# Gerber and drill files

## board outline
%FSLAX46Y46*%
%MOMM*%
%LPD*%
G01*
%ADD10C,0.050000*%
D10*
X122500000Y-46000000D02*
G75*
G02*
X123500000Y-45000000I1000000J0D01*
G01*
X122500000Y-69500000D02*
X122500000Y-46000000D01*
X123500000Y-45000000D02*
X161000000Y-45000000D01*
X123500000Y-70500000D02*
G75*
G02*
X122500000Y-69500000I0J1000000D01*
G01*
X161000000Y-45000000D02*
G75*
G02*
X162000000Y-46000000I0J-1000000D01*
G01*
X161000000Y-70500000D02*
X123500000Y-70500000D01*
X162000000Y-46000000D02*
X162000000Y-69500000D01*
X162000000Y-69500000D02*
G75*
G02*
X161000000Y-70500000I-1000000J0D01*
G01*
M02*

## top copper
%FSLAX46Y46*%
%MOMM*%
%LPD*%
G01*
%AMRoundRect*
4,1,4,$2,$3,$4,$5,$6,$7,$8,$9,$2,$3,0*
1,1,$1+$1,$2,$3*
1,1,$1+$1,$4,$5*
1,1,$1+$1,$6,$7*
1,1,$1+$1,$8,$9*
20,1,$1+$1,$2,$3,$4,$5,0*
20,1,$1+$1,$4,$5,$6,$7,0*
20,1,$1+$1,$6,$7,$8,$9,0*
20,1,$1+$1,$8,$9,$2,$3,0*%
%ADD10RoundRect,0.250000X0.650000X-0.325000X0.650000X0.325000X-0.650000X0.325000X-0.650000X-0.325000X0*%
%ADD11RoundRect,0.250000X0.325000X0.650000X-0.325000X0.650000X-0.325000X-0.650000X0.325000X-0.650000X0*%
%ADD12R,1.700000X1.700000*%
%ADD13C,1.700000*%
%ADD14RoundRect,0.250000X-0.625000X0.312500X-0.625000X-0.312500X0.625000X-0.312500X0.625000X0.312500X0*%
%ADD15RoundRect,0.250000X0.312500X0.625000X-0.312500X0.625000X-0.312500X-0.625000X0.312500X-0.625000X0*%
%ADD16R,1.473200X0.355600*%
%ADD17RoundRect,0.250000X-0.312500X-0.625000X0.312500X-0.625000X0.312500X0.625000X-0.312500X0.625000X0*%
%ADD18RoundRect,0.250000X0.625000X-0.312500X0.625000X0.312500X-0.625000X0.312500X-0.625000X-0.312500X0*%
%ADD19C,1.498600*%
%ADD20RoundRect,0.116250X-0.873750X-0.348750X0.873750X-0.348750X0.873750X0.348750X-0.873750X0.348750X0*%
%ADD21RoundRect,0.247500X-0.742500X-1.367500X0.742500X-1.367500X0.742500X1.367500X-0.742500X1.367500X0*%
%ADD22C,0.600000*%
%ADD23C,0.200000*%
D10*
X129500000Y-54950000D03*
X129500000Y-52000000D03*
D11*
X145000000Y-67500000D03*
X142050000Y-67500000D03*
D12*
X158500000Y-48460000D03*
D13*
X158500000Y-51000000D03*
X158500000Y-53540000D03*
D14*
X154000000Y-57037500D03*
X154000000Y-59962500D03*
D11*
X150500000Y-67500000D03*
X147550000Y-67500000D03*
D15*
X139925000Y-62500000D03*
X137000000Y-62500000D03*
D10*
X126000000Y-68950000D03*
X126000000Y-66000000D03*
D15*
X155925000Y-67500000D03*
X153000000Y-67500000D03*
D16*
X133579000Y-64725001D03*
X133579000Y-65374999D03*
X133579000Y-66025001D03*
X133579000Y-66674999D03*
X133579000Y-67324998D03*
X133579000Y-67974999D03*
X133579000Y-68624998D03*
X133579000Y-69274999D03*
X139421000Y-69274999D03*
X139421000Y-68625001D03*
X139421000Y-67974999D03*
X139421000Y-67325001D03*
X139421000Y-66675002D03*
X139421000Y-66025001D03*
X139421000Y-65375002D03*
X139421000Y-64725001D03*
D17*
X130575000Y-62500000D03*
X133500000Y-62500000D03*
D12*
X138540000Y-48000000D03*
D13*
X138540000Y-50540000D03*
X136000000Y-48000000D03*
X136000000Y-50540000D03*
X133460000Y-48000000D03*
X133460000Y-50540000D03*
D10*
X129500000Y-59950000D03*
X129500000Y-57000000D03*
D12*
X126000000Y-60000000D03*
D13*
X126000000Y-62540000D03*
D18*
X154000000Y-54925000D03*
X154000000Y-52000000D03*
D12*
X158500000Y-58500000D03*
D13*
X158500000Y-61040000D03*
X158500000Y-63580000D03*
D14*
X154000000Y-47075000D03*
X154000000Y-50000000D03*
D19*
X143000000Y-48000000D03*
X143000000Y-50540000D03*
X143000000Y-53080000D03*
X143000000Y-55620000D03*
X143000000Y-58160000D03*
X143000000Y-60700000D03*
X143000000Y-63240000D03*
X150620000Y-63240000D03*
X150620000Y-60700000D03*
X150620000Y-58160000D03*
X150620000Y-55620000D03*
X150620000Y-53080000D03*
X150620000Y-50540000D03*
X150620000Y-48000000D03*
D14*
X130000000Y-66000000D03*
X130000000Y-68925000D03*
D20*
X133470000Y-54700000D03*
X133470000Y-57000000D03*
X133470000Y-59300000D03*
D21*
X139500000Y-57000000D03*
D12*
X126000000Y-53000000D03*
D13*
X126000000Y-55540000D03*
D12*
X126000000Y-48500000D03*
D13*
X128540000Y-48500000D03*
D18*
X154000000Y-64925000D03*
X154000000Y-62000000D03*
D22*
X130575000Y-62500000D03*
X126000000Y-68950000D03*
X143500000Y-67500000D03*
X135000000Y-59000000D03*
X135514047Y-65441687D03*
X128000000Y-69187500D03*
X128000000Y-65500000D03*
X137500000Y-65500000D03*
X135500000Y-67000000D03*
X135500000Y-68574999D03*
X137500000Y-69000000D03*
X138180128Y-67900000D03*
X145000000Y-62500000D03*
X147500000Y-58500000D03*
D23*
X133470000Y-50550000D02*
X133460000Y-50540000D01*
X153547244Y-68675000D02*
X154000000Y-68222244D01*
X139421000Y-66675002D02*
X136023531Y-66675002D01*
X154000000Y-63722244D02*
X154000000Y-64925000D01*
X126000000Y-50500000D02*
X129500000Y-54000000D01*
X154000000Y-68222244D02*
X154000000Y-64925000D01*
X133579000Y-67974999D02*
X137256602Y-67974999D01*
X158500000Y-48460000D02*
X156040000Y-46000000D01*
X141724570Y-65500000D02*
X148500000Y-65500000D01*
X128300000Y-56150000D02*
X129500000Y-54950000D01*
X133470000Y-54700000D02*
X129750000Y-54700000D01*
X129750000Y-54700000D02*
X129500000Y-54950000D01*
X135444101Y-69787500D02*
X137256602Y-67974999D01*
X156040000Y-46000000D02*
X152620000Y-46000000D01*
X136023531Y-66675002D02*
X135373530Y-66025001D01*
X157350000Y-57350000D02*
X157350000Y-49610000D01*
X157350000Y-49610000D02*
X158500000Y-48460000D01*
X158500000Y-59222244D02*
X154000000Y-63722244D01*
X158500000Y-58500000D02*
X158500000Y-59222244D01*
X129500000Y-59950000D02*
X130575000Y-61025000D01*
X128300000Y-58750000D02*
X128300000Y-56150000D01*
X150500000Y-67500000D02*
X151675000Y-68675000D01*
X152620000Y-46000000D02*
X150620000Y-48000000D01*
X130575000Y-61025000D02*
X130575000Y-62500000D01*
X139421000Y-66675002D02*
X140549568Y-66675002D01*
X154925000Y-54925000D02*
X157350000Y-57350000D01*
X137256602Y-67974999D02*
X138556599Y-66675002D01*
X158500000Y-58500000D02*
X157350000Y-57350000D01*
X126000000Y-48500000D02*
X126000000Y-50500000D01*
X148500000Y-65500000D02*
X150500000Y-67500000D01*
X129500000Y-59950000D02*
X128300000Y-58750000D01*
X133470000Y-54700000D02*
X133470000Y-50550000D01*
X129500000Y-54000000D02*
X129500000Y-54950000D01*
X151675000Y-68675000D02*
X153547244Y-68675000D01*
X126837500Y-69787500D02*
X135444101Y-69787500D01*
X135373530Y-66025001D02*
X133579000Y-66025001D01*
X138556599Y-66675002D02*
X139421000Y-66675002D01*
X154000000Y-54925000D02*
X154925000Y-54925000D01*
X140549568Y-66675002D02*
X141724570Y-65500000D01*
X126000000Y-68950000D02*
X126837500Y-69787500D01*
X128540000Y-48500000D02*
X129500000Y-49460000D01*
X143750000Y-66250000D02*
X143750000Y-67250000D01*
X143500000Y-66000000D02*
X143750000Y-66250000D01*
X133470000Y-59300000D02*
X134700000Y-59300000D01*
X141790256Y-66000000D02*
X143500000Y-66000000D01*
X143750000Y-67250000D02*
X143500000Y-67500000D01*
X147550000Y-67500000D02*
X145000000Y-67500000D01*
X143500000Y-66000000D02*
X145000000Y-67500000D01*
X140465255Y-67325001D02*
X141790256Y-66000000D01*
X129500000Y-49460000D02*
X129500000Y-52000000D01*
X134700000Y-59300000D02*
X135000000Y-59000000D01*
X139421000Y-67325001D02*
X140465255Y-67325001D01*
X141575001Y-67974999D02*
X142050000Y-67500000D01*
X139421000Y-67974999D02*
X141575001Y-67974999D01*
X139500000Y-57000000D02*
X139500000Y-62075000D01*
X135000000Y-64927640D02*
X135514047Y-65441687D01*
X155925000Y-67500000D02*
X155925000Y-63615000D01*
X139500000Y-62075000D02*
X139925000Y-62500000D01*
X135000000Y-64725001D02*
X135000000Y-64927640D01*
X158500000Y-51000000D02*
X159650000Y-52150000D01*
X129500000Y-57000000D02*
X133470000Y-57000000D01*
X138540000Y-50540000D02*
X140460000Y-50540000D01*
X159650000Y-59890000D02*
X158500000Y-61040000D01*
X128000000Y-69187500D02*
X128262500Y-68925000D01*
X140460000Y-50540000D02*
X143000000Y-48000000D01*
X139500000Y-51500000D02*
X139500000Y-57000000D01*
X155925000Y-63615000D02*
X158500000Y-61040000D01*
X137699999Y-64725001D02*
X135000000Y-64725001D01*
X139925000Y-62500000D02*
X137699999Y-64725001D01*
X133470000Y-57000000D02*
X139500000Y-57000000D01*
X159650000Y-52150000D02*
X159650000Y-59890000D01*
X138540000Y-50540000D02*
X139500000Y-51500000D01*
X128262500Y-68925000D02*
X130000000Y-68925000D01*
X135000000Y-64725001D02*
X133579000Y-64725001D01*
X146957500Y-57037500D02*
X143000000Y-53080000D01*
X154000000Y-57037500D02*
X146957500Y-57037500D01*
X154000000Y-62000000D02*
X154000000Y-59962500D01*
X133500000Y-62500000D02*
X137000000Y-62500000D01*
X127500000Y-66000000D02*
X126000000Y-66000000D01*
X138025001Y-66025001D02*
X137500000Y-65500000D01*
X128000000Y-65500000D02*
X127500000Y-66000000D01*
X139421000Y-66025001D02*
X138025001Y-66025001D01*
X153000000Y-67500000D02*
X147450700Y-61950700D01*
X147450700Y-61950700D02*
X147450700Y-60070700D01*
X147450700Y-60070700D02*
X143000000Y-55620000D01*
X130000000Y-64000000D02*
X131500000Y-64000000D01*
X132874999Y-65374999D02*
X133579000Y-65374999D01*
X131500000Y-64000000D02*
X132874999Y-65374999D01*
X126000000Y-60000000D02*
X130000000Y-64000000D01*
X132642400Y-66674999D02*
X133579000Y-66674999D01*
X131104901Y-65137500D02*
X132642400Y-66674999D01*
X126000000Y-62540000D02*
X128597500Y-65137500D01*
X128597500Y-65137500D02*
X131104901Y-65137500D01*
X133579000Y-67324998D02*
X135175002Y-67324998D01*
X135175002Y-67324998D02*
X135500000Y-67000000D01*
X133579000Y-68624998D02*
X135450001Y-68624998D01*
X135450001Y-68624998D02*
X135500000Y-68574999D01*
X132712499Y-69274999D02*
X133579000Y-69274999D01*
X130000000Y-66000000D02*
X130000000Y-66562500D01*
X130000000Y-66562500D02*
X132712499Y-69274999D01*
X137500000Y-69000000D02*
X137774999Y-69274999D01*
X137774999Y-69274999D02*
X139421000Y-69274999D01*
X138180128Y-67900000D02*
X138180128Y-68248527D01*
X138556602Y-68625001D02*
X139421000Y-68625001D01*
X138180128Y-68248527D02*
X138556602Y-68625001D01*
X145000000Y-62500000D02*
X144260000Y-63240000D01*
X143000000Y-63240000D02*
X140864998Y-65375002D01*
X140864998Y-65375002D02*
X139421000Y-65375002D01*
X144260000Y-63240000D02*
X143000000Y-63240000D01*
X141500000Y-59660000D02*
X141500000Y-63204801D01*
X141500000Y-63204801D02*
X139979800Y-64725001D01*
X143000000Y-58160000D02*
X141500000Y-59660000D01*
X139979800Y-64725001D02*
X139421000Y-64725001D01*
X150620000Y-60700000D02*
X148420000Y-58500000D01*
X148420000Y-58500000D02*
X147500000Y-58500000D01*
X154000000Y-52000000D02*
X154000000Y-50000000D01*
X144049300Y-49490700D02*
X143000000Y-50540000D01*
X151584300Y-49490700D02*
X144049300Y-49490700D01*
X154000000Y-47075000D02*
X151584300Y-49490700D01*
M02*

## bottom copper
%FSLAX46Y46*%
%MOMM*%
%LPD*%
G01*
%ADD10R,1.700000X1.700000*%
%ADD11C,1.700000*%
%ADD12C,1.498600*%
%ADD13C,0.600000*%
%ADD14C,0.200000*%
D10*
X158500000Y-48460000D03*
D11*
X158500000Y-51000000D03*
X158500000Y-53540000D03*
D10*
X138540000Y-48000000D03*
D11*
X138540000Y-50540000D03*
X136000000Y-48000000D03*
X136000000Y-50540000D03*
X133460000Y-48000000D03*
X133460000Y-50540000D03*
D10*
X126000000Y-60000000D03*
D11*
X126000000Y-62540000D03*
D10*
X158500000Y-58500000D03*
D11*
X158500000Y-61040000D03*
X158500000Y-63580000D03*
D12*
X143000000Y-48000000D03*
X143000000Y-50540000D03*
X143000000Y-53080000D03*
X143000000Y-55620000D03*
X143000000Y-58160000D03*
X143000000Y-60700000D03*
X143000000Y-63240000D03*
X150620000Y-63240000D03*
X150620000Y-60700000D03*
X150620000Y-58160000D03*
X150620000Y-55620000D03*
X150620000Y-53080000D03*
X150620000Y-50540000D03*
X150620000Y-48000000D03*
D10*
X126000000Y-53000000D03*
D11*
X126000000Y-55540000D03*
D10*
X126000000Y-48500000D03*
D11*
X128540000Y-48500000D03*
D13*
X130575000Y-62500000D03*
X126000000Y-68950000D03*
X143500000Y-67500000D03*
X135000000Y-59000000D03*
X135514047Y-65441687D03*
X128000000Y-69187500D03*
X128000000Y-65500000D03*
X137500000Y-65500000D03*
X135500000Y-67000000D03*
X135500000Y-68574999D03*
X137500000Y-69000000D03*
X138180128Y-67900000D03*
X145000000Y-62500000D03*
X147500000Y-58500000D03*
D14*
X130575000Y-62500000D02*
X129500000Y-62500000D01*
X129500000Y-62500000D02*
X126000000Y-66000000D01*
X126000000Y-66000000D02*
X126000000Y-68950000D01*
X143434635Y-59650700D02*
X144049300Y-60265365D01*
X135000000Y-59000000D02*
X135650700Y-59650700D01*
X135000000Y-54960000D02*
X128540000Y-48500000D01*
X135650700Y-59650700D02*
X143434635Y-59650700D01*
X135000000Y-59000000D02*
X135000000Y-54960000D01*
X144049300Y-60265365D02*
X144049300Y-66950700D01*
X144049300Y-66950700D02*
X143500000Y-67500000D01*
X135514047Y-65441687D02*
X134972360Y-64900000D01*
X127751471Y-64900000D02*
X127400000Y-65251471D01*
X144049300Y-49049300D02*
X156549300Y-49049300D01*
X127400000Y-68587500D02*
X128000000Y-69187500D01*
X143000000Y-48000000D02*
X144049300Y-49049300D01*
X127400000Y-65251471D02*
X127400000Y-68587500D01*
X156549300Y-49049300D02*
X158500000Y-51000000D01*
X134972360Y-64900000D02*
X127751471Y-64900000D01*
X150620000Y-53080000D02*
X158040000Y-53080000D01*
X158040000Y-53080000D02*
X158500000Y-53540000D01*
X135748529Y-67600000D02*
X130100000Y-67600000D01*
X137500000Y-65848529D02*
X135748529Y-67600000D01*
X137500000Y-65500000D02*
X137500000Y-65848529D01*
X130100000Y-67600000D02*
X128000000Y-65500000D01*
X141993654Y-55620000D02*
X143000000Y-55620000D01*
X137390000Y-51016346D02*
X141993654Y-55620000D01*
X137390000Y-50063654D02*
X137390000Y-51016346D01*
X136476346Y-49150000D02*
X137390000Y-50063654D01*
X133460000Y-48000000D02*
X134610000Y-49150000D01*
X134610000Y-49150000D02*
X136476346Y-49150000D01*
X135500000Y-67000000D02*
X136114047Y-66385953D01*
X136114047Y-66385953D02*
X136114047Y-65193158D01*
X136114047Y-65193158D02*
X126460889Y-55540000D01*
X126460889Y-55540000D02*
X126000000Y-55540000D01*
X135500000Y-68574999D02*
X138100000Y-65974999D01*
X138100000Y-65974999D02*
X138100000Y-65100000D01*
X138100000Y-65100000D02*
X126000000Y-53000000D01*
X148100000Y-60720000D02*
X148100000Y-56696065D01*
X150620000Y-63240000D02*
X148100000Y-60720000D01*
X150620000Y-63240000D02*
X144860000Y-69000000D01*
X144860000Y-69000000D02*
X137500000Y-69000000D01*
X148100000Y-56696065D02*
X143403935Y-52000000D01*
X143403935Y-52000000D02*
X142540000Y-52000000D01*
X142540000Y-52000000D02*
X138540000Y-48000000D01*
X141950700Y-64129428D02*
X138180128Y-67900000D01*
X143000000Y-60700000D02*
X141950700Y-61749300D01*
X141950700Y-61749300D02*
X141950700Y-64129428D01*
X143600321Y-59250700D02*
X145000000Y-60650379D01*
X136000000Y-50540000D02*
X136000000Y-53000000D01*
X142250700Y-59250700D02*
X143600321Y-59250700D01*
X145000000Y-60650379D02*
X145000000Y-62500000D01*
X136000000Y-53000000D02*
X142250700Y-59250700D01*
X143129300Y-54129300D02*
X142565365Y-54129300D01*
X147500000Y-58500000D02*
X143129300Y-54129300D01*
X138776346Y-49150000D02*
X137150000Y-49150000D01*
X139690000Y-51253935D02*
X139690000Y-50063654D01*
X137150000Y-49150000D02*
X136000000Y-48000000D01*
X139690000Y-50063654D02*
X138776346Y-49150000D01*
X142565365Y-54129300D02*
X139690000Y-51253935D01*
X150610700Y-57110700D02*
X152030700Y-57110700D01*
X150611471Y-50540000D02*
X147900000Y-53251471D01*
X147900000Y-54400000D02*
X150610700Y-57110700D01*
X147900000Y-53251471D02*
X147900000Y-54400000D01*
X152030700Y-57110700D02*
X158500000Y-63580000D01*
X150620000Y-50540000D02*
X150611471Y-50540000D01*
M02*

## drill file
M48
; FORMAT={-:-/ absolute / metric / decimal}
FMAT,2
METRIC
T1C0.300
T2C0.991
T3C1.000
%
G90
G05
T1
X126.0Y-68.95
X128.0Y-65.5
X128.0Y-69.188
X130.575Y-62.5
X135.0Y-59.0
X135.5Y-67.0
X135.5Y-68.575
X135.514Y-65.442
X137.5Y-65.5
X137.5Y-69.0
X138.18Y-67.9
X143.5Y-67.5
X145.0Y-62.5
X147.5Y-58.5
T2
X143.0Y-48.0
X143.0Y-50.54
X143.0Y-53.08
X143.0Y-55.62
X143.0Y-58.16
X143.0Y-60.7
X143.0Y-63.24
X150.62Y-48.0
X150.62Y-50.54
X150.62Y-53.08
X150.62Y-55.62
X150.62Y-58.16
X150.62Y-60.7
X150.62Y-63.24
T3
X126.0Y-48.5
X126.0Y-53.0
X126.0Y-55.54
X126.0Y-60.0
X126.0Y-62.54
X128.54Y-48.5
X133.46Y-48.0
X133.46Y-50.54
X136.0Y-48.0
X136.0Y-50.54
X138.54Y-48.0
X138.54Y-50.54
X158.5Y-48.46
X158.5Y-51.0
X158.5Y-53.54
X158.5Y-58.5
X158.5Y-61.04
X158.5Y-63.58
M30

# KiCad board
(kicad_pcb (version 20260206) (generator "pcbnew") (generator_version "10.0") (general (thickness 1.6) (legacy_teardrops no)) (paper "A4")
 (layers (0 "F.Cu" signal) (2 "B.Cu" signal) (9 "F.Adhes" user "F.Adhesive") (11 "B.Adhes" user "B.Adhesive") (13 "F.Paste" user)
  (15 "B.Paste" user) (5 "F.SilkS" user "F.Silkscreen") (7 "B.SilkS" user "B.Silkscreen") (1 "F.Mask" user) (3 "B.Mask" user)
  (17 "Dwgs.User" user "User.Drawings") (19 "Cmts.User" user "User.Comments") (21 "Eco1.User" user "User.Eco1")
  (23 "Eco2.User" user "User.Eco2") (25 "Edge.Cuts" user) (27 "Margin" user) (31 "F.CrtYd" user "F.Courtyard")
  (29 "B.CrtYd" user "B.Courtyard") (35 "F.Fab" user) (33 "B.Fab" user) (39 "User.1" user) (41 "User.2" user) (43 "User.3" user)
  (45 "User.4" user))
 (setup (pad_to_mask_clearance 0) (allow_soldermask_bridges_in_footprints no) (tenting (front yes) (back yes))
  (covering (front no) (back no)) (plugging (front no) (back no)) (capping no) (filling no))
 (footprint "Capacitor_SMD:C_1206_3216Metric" (layer "F.Cu") (at 129.5 53.475 90)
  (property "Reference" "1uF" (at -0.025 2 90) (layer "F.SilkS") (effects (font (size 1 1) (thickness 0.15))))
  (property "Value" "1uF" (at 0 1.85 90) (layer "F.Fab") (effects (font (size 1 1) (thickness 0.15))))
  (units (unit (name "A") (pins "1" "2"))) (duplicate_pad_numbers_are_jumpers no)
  (pad "1" smd roundrect (at -1.475 0 90) (size 1.15 1.8) (layers "F.Cu" "F.Mask" "F.Paste") (roundrect_rratio 0.217391) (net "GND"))
  (pad "2" smd roundrect (at 1.475 0 90) (size 1.15 1.8) (layers "F.Cu" "F.Mask" "F.Paste") (roundrect_rratio 0.217391) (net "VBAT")))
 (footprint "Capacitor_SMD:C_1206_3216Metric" (layer "F.Cu") (at 143.525 67.5 180)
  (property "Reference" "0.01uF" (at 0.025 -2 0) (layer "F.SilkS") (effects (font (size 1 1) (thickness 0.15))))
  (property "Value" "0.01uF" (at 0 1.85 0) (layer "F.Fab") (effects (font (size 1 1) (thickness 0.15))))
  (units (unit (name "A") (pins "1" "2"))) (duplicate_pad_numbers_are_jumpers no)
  (pad "1" smd roundrect (at -1.475 0 180) (size 1.15 1.8) (layers "F.Cu" "F.Mask" "F.Paste") (roundrect_rratio 0.217391) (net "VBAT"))
  (pad "2" smd roundrect (at 1.475 0 180) (size 1.15 1.8) (layers "F.Cu" "F.Mask" "F.Paste") (roundrect_rratio 0.217391)
   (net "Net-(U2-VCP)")))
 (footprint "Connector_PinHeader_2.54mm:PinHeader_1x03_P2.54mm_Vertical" (layer "F.Cu") (at 158.5 48.46)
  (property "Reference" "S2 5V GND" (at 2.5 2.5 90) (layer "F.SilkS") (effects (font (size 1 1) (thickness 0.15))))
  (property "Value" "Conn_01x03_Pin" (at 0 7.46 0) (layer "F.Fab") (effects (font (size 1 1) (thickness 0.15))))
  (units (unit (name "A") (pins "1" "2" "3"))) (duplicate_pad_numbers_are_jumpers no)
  (pad "1" thru_hole rect (at 0 0) (size 1.7 1.7) (drill 1) (layers "*.Cu" "*.Mask") (remove_unused_layers no) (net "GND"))
  (pad "2" thru_hole circle (at 0 2.54) (size 1.7 1.7) (drill 1) (layers "*.Cu" "*.Mask") (remove_unused_layers no) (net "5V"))
  (pad "3" thru_hole circle (at 0 5.08) (size 1.7 1.7) (drill 1) (layers "*.Cu" "*.Mask") (remove_unused_layers no)
   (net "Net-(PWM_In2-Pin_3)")))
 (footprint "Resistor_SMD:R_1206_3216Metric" (layer "F.Cu") (at 154 58.5 -90)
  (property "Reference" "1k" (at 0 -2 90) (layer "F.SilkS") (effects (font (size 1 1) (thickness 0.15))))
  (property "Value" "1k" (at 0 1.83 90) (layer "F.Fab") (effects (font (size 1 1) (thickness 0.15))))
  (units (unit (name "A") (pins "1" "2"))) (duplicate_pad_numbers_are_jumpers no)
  (pad "1" smd roundrect (at -1.4625 0 270) (size 1.125 1.75) (layers "F.Cu" "F.Mask" "F.Paste") (roundrect_rratio 0.222222)
   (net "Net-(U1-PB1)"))
  (pad "2" smd roundrect (at 1.4625 0 270) (size 1.125 1.75) (layers "F.Cu" "F.Mask" "F.Paste") (roundrect_rratio 0.222222)
   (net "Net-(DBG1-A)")))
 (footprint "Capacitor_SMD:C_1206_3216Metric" (layer "F.Cu") (at 149.025 67.5 180)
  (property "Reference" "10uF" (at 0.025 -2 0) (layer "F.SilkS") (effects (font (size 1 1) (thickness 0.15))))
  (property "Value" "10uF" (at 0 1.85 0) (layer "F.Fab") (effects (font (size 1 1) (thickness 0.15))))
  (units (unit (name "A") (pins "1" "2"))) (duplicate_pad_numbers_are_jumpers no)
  (pad "1" smd roundrect (at -1.475 0 180) (size 1.15 1.8) (layers "F.Cu" "F.Mask" "F.Paste") (roundrect_rratio 0.217391) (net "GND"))
  (pad "2" smd roundrect (at 1.475 0 180) (size 1.15 1.8) (layers "F.Cu" "F.Mask" "F.Paste") (roundrect_rratio 0.217391) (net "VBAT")))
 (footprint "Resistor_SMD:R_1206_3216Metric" (layer "F.Cu") (at 138.4625 62.5 180)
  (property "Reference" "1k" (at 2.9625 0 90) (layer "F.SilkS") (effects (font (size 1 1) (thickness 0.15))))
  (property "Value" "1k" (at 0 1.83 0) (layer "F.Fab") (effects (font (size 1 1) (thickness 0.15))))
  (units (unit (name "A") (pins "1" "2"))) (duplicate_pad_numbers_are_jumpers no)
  (pad "1" smd roundrect (at -1.4625 0 180) (size 1.125 1.75) (layers "F.Cu" "F.Mask" "F.Paste") (roundrect_rratio 0.222222) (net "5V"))
  (pad "2" smd roundrect (at 1.4625 0 180) (size 1.125 1.75) (layers "F.Cu" "F.Mask" "F.Paste") (roundrect_rratio 0.222222)
   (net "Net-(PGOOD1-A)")))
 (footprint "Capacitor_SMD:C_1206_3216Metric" (layer "F.Cu") (at 126 67.475 90)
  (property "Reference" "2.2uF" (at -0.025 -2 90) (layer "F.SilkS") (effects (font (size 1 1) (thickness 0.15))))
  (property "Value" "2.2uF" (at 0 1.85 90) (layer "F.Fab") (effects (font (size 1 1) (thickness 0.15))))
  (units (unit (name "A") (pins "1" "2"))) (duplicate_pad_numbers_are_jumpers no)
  (pad "1" smd roundrect (at -1.475 0 90) (size 1.15 1.8) (layers "F.Cu" "F.Mask" "F.Paste") (roundrect_rratio 0.217391) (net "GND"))
  (pad "2" smd roundrect (at 1.475 0 90) (size 1.15 1.8) (layers "F.Cu" "F.Mask" "F.Paste") (roundrect_rratio 0.217391)
   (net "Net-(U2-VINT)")))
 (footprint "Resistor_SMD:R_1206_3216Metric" (layer "F.Cu") (at 154.4625 67.5 180)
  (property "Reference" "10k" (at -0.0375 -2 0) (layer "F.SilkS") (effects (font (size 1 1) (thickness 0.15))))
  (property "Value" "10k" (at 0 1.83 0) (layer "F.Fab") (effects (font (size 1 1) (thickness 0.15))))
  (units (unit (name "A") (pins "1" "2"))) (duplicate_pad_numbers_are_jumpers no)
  (pad "1" smd roundrect (at -1.4625 0 180) (size 1.125 1.75) (layers "F.Cu" "F.Mask" "F.Paste") (roundrect_rratio 0.222222) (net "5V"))
  (pad "2" smd roundrect (at 1.4625 0 180) (size 1.125 1.75) (layers "F.Cu" "F.Mask" "F.Paste") (roundrect_rratio 0.222222) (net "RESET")))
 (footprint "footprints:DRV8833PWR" (layer "F.Cu") (at 136.5 67)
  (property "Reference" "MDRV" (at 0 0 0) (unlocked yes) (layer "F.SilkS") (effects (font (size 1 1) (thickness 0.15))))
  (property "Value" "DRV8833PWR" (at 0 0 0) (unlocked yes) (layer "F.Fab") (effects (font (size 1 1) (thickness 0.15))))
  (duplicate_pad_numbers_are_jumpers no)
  (pad "1" smd rect (at -2.921 -2.274999) (size 1.4732 0.3556) (layers "F.Cu" "F.Mask" "F.Paste") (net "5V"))
  (pad "2" smd rect (at -2.921 -1.625001) (size 1.4732 0.3556) (layers "F.Cu" "F.Mask" "F.Paste") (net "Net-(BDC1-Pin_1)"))
  (pad "3" smd rect (at -2.921 -0.974999) (size 1.4732 0.3556) (layers "F.Cu" "F.Mask" "F.Paste") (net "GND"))
  (pad "4" smd rect (at -2.921 -0.325001) (size 1.4732 0.3556) (layers "F.Cu" "F.Mask" "F.Paste") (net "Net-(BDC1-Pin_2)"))
  (pad "5" smd rect (at -2.921 0.324998) (size 1.4732 0.3556) (layers "F.Cu" "F.Mask" "F.Paste") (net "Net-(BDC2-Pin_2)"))
  (pad "6" smd rect (at -2.921 0.974999) (size 1.4732 0.3556) (layers "F.Cu" "F.Mask" "F.Paste") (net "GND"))
  (pad "7" smd rect (at -2.921 1.624998) (size 1.4732 0.3556) (layers "F.Cu" "F.Mask" "F.Paste") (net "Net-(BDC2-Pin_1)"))
  (pad "8" smd rect (at -2.921 2.274999) (size 1.4732 0.3556) (layers "F.Cu" "F.Mask" "F.Paste") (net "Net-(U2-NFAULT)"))
  (pad "9" smd rect (at 2.921 2.274999) (size 1.4732 0.3556) (layers "F.Cu" "F.Mask" "F.Paste") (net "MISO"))
  (pad "10" smd rect (at 2.921 1.625001) (size 1.4732 0.3556) (layers "F.Cu" "F.Mask" "F.Paste") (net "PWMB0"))
  (pad "11" smd rect (at 2.921 0.974999) (size 1.4732 0.3556) (layers "F.Cu" "F.Mask" "F.Paste") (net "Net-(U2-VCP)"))
  (pad "12" smd rect (at 2.921 0.325001) (size 1.4732 0.3556) (layers "F.Cu" "F.Mask" "F.Paste") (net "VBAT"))
  (pad "13" smd rect (at 2.921 -0.324998) (size 1.4732 0.3556) (layers "F.Cu" "F.Mask" "F.Paste") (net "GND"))
  (pad "14" smd rect (at 2.921 -0.974999) (size 1.4732 0.3556) (layers "F.Cu" "F.Mask" "F.Paste") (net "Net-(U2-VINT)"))
  (pad "15" smd rect (at 2.921 -1.624998) (size 1.4732 0.3556) (layers "F.Cu" "F.Mask" "F.Paste") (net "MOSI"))
  (pad "16" smd rect (at 2.921 -2.274999) (size 1.4732 0.3556) (layers "F.Cu" "F.Mask" "F.Paste") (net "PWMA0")))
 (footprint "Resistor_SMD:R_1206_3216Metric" (layer "F.Cu") (at 132.0375 62.5)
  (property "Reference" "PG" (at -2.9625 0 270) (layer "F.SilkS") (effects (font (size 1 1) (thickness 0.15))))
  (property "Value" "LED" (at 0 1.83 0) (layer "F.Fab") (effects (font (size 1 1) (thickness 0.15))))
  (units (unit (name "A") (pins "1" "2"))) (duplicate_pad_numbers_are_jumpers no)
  (pad "1" smd roundrect (at -1.4625 0) (size 1.125 1.75) (layers "F.Cu" "F.Mask" "F.Paste") (roundrect_rratio 0.222222) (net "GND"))
  (pad "2" smd roundrect (at 1.4625 0) (size 1.125 1.75) (layers "F.Cu" "F.Mask" "F.Paste") (roundrect_rratio 0.222222)
   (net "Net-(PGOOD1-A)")))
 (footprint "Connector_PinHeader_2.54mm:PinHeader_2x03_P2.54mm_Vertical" (layer "F.Cu") (at 138.54 48 -90)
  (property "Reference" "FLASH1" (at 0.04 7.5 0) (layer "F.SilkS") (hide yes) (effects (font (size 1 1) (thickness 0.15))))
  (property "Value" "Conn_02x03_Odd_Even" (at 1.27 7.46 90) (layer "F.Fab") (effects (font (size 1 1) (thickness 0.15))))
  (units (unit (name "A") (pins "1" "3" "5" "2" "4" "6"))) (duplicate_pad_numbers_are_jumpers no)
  (pad "1" thru_hole rect (at 0 0 270) (size 1.7 1.7) (drill 1) (layers "*.Cu" "*.Mask") (remove_unused_layers no) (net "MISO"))
  (pad "2" thru_hole circle (at 2.54 0 270) (size 1.7 1.7) (drill 1) (layers "*.Cu" "*.Mask") (remove_unused_layers no) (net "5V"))
  (pad "3" thru_hole circle (at 0 2.54 270) (size 1.7 1.7) (drill 1) (layers "*.Cu" "*.Mask") (remove_unused_layers no) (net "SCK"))
  (pad "4" thru_hole circle (at 2.54 2.54 270) (size 1.7 1.7) (drill 1) (layers "*.Cu" "*.Mask") (remove_unused_layers no) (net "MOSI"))
  (pad "5" thru_hole circle (at 0 5.08 270) (size 1.7 1.7) (drill 1) (layers "*.Cu" "*.Mask") (remove_unused_layers no) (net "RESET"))
  (pad "6" thru_hole circle (at 2.54 5.08 270) (size 1.7 1.7) (drill 1) (layers "*.Cu" "*.Mask") (remove_unused_layers no) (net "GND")))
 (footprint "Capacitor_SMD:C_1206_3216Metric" (layer "F.Cu") (at 129.5 58.475 90)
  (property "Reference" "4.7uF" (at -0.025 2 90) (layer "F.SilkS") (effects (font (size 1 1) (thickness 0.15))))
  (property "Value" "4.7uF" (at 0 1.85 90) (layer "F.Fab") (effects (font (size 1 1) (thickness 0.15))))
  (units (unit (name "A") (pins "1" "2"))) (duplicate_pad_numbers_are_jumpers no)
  (pad "1" smd roundrect (at -1.475 0 90) (size 1.15 1.8) (layers "F.Cu" "F.Mask" "F.Paste") (roundrect_rratio 0.217391) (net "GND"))
  (pad "2" smd roundrect (at 1.475 0 90) (size 1.15 1.8) (layers "F.Cu" "F.Mask" "F.Paste") (roundrect_rratio 0.217391) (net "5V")))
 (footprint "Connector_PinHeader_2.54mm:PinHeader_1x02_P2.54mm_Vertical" (layer "F.Cu") (at 126 60)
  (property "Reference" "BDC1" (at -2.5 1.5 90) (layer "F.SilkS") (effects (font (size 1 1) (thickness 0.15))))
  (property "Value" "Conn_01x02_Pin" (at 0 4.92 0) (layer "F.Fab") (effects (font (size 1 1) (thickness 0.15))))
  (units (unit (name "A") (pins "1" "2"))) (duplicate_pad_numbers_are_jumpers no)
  (pad "1" thru_hole rect (at 0 0) (size 1.7 1.7) (drill 1) (layers "*.Cu" "*.Mask") (remove_unused_layers no) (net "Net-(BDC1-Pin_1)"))
  (pad "2" thru_hole circle (at 0 2.54) (size 1.7 1.7) (drill 1) (layers "*.Cu" "*.Mask") (remove_unused_layers no) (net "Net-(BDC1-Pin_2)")))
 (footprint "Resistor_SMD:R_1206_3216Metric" (layer "F.Cu") (at 154 53.4625 90)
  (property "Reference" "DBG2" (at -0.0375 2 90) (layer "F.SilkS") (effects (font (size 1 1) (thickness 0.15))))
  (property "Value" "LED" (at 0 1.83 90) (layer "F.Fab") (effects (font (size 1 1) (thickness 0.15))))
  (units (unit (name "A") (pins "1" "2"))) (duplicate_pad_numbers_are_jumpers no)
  (pad "1" smd roundrect (at -1.4625 0 90) (size 1.125 1.75) (layers "F.Cu" "F.Mask" "F.Paste") (roundrect_rratio 0.222222) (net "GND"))
  (pad "2" smd roundrect (at 1.4625 0 90) (size 1.125 1.75) (layers "F.Cu" "F.Mask" "F.Paste") (roundrect_rratio 0.222222)
   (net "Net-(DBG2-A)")))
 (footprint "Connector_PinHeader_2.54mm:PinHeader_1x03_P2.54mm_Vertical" (layer "F.Cu") (at 158.5 58.5)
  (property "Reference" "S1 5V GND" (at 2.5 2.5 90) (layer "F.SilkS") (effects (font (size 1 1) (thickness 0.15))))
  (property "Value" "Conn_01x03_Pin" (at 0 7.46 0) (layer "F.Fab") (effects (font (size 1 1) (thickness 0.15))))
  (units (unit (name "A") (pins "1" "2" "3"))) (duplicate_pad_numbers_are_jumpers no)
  (pad "1" thru_hole rect (at 0 0) (size 1.7 1.7) (drill 1) (layers "*.Cu" "*.Mask") (remove_unused_layers no) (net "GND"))
  (pad "2" thru_hole circle (at 0 2.54) (size 1.7 1.7) (drill 1) (layers "*.Cu" "*.Mask") (remove_unused_layers no) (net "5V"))
  (pad "3" thru_hole circle (at 0 5.08) (size 1.7 1.7) (drill 1) (layers "*.Cu" "*.Mask") (remove_unused_layers no)
   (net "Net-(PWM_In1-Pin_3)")))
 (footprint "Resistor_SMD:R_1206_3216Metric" (layer "F.Cu") (at 154 48.5375 -90)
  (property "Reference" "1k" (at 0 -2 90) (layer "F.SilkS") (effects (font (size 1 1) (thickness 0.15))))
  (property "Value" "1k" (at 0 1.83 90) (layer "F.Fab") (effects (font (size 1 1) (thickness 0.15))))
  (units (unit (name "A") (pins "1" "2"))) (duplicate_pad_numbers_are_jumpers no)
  (pad "1" smd roundrect (at -1.4625 0 270) (size 1.125 1.75) (layers "F.Cu" "F.Mask" "F.Paste") (roundrect_rratio 0.222222)
   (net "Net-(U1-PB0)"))
  (pad "2" smd roundrect (at 1.4625 0 270) (size 1.125 1.75) (layers "F.Cu" "F.Mask" "F.Paste") (roundrect_rratio 0.222222)
   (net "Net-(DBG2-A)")))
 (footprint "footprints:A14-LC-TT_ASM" (layer "F.Cu") (at 150.62 48 -90)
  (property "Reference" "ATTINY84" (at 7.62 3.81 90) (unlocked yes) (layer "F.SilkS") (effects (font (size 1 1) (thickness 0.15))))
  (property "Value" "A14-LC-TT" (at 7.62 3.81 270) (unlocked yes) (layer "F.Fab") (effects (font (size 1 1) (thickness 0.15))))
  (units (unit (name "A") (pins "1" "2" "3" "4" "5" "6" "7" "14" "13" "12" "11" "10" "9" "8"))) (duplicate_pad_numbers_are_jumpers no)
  (pad "1" thru_hole circle (at 0 7.62 270) (size 1.4986 1.4986) (drill 0.9906) (layers "*.Cu" "*.Mask") (remove_unused_layers no)
   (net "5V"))
  (pad "2" thru_hole circle (at 2.54 7.62 270) (size 1.4986 1.4986) (drill 0.9906) (layers "*.Cu" "*.Mask") (remove_unused_layers no)
   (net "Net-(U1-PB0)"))
  (pad "3" thru_hole circle (at 5.08 7.62 270) (size 1.4986 1.4986) (drill 0.9906) (layers "*.Cu" "*.Mask") (remove_unused_layers no)
   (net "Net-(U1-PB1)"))
  (pad "4" thru_hole circle (at 7.62 7.62 270) (size 1.4986 1.4986) (drill 0.9906) (layers "*.Cu" "*.Mask") (remove_unused_layers no)
   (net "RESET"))
  (pad "5" thru_hole circle (at 10.16 7.62 270) (size 1.4986 1.4986) (drill 0.9906) (layers "*.Cu" "*.Mask") (remove_unused_layers no)
   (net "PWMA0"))
  (pad "6" thru_hole circle (at 12.7 7.62 270) (size 1.4986 1.4986) (drill 0.9906) (layers "*.Cu" "*.Mask") (remove_unused_layers no)
   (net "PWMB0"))
  (pad "7" thru_hole circle (at 15.24 7.62 270) (size 1.4986 1.4986) (drill 0.9906) (layers "*.Cu" "*.Mask") (remove_unused_layers no)
   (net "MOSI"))
  (pad "8" thru_hole circle (at 15.24 0 270) (size 1.4986 1.4986) (drill 0.9906) (layers "*.Cu" "*.Mask") (remove_unused_layers no)
   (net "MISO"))
  (pad "9" thru_hole circle (at 12.7 0 270) (size 1.4986 1.4986) (drill 0.9906) (layers "*.Cu" "*.Mask") (remove_unused_layers no)
   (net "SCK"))
  (pad "10" thru_hole circle (at 10.16 0 270) (size 1.4986 1.4986) (drill 0.9906) (layers "*.Cu" "*.Mask") (remove_unused_layers no)
   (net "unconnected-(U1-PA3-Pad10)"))
  (pad "11" thru_hole circle (at 7.62 0 270) (size 1.4986 1.4986) (drill 0.9906) (layers "*.Cu" "*.Mask") (remove_unused_layers no)
   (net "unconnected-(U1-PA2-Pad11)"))
  (pad "12" thru_hole circle (at 5.08 0 270) (size 1.4986 1.4986) (drill 0.9906) (layers "*.Cu" "*.Mask") (remove_unused_layers no)
   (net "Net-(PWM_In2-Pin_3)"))
  (pad "13" thru_hole circle (at 2.54 0 270) (size 1.4986 1.4986) (drill 0.9906) (layers "*.Cu" "*.Mask") (remove_unused_layers no)
   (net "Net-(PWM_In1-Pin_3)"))
  (pad "14" thru_hole circle (at 0 0 270) (size 1.4986 1.4986) (drill 0.9906) (layers "*.Cu" "*.Mask") (remove_unused_layers no) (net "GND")))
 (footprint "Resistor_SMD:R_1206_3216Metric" (layer "F.Cu") (at 130 67.4625 -90)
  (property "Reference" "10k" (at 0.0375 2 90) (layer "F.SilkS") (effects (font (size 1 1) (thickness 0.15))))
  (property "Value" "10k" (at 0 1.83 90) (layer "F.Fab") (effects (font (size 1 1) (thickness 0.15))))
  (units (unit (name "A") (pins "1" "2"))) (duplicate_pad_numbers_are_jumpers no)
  (pad "1" smd roundrect (at -1.4625 0 270) (size 1.125 1.75) (layers "F.Cu" "F.Mask" "F.Paste") (roundrect_rratio 0.222222)
   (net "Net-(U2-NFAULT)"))
  (pad "2" smd roundrect (at 1.4625 0 270) (size 1.125 1.75) (layers "F.Cu" "F.Mask" "F.Paste") (roundrect_rratio 0.222222) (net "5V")))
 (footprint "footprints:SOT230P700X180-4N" (layer "F.Cu") (at 136.485 57)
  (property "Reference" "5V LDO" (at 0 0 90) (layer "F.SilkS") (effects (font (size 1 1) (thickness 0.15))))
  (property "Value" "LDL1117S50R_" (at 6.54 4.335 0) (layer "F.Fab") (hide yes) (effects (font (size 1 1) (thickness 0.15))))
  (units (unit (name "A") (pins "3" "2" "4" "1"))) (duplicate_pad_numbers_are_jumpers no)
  (pad "1" smd roundrect (at -3.015 -2.3) (size 1.98 0.93) (layers "F.Cu" "F.Mask" "F.Paste") (roundrect_rratio 0.125) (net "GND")
   (solder_mask_margin 0.102))
  (pad "2" smd roundrect (at -3.015 0) (size 1.98 0.93) (layers "F.Cu" "F.Mask" "F.Paste") (roundrect_rratio 0.125) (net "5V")
   (solder_mask_margin 0.102))
  (pad "3" smd roundrect (at -3.015 2.3) (size 1.98 0.93) (layers "F.Cu" "F.Mask" "F.Paste") (roundrect_rratio 0.125) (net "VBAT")
   (solder_mask_margin 0.102))
  (pad "4" smd roundrect (at 3.015 0) (size 1.98 3.23) (layers "F.Cu" "F.Mask" "F.Paste") (roundrect_rratio 0.125) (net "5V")
   (solder_mask_margin 0.102)))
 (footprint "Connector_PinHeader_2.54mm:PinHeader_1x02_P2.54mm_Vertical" (layer "F.Cu") (at 126 53)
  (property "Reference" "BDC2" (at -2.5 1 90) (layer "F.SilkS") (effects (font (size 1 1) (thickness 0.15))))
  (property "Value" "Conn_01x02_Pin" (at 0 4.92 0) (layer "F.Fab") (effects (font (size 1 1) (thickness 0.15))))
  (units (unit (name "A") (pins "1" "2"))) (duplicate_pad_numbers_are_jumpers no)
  (pad "1" thru_hole rect (at 0 0) (size 1.7 1.7) (drill 1) (layers "*.Cu" "*.Mask") (remove_unused_layers no) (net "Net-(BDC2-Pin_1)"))
  (pad "2" thru_hole circle (at 0 2.54) (size 1.7 1.7) (drill 1) (layers "*.Cu" "*.Mask") (remove_unused_layers no) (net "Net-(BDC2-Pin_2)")))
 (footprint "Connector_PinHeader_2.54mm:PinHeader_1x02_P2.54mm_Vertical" (layer "F.Cu") (at 126 48.5 90)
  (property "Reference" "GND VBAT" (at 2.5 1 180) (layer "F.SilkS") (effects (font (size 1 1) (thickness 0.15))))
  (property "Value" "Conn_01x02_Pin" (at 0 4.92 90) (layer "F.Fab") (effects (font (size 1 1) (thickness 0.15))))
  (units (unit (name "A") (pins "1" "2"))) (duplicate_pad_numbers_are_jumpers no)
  (pad "1" thru_hole rect (at 0 0 90) (size 1.7 1.7) (drill 1) (layers "*.Cu" "*.Mask") (remove_unused_layers no) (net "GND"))
  (pad "2" thru_hole circle (at 0 2.54 90) (size 1.7 1.7) (drill 1) (layers "*.Cu" "*.Mask") (remove_unused_layers no) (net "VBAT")))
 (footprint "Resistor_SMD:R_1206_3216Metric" (layer "F.Cu") (at 154 63.4625 90)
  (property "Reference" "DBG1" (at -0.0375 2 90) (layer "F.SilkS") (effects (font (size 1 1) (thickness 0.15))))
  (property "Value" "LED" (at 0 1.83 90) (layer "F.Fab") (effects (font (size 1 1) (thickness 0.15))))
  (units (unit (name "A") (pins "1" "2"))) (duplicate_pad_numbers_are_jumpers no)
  (pad "1" smd roundrect (at -1.4625 0 90) (size 1.125 1.75) (layers "F.Cu" "F.Mask" "F.Paste") (roundrect_rratio 0.222222) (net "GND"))
  (pad "2" smd roundrect (at 1.4625 0 90) (size 1.125 1.75) (layers "F.Cu" "F.Mask" "F.Paste") (roundrect_rratio 0.222222)
   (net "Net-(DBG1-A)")))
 (gr_arc (start 122.5 46) (mid 122.792893 45.292893) (end 123.5 45) (stroke (width 0.05) (type default)) (layer "Edge.Cuts"))
 (gr_line (start 122.5 69.5) (end 122.5 46) (stroke (width 0.05) (type default)) (layer "Edge.Cuts"))
 (gr_line (start 123.5 45) (end 161 45) (stroke (width 0.05) (type default)) (layer "Edge.Cuts"))
 (gr_arc (start 123.5 70.5) (mid 122.792893 70.207107) (end 122.5 69.5) (stroke (width 0.05) (type default)) (layer "Edge.Cuts"))
 (gr_arc (start 161 45) (mid 161.707107 45.292893) (end 162 46) (stroke (width 0.05) (type default)) (layer "Edge.Cuts"))
 (gr_line (start 161 70.5) (end 123.5 70.5) (stroke (width 0.05) (type default)) (layer "Edge.Cuts"))
 (gr_line (start 162 46) (end 162 69.5) (stroke (width 0.05) (type default)) (layer "Edge.Cuts"))
 (gr_arc (start 162 69.5) (mid 161.707107 70.207107) (end 161 70.5) (stroke (width 0.05) (type default)) (layer "Edge.Cuts"))
 (segment (start 133.47 50.55) (end 133.46 50.54) (width 0.2) (layer "F.Cu") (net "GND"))
 (segment (start 153.547244 68.675) (end 154 68.222244) (width 0.2) (layer "F.Cu") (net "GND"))
 (segment (start 139.421 66.675002) (end 136.023531 66.675002) (width 0.2) (layer "F.Cu") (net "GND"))
 (segment (start 154 63.722244) (end 154 64.925) (width 0.2) (layer "F.Cu") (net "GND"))
 (segment (start 126 50.5) (end 129.5 54) (width 0.2) (layer "F.Cu") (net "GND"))
 (segment (start 154 68.222244) (end 154 64.925) (width 0.2) (layer "F.Cu") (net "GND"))
 (segment (start 133.579 67.974999) (end 137.256602 67.974999) (width 0.2) (layer "F.Cu") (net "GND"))
 (segment (start 158.5 48.46) (end 156.04 46) (width 0.2) (layer "F.Cu") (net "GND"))
 (segment (start 141.72457 65.5) (end 148.5 65.5) (width 0.2) (layer "F.Cu") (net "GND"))
 (segment (start 128.3 56.15) (end 129.5 54.95) (width 0.2) (layer "F.Cu") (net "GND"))
 (segment (start 133.47 54.7) (end 129.75 54.7) (width 0.2) (layer "F.Cu") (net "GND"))
 (segment (start 129.75 54.7) (end 129.5 54.95) (width 0.2) (layer "F.Cu") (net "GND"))
 (segment (start 135.444101 69.7875) (end 137.256602 67.974999) (width 0.2) (layer "F.Cu") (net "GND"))
 (segment (start 156.04 46) (end 152.62 46) (width 0.2) (layer "F.Cu") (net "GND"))
 (segment (start 136.023531 66.675002) (end 135.37353 66.025001) (width 0.2) (layer "F.Cu") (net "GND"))
 (segment (start 157.35 57.35) (end 157.35 49.61) (width 0.2) (layer "F.Cu") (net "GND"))
 (segment (start 157.35 49.61) (end 158.5 48.46) (width 0.2) (layer "F.Cu") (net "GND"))
 (segment (start 158.5 59.222244) (end 154 63.722244) (width 0.2) (layer "F.Cu") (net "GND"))
 (segment (start 158.5 58.5) (end 158.5 59.222244) (width 0.2) (layer "F.Cu") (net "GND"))
 (segment (start 129.5 59.95) (end 130.575 61.025) (width 0.2) (layer "F.Cu") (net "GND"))
 (segment (start 128.3 58.75) (end 128.3 56.15) (width 0.2) (layer "F.Cu") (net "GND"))
 (segment (start 150.5 67.5) (end 151.675 68.675) (width 0.2) (layer "F.Cu") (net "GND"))
 (segment (start 152.62 46) (end 150.62 48) (width 0.2) (layer "F.Cu") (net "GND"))
 (segment (start 130.575 61.025) (end 130.575 62.5) (width 0.2) (layer "F.Cu") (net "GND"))
 (segment (start 139.421 66.675002) (end 140.549568 66.675002) (width 0.2) (layer "F.Cu") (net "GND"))
 (segment (start 154.925 54.925) (end 157.35 57.35) (width 0.2) (layer "F.Cu") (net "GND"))
 (segment (start 137.256602 67.974999) (end 138.556599 66.675002) (width 0.2) (layer "F.Cu") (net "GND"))
 (segment (start 158.5 58.5) (end 157.35 57.35) (width 0.2) (layer "F.Cu") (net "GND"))
 (segment (start 126 48.5) (end 126 50.5) (width 0.2) (layer "F.Cu") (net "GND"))
 (segment (start 148.5 65.5) (end 150.5 67.5) (width 0.2) (layer "F.Cu") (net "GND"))
 (segment (start 129.5 59.95) (end 128.3 58.75) (width 0.2) (layer "F.Cu") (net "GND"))
 (segment (start 133.47 54.7) (end 133.47 50.55) (width 0.2) (layer "F.Cu") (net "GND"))
 (segment (start 129.5 54) (end 129.5 54.95) (width 0.2) (layer "F.Cu") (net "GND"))
 (segment (start 151.675 68.675) (end 153.547244 68.675) (width 0.2) (layer "F.Cu") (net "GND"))
 (segment (start 126.8375 69.7875) (end 135.444101 69.7875) (width 0.2) (layer "F.Cu") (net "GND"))
 (segment (start 135.37353 66.025001) (end 133.579 66.025001) (width 0.2) (layer "F.Cu") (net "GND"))
 (segment (start 138.556599 66.675002) (end 139.421 66.675002) (width 0.2) (layer "F.Cu") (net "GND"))
 (segment (start 154 54.925) (end 154.925 54.925) (width 0.2) (layer "F.Cu") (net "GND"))
 (segment (start 140.549568 66.675002) (end 141.72457 65.5) (width 0.2) (layer "F.Cu") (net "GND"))
 (segment (start 126 68.95) (end 126.8375 69.7875) (width 0.2) (layer "F.Cu") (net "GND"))
 (via (at 130.575 62.5) (size 0.6) (drill 0.3) (layers "F.Cu" "B.Cu") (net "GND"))
 (via (at 126 68.95) (size 0.6) (drill 0.3) (layers "F.Cu" "B.Cu") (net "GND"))
 (segment (start 130.575 62.5) (end 129.5 62.5) (width 0.2) (layer "B.Cu") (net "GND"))
 (segment (start 129.5 62.5) (end 126 66) (width 0.2) (layer "B.Cu") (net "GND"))
 (segment (start 126 66) (end 126 68.95) (width 0.2) (layer "B.Cu") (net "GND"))
 (segment (start 128.54 48.5) (end 129.5 49.46) (width 0.2) (layer "F.Cu") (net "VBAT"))
 (segment (start 143.75 66.25) (end 143.75 67.25) (width 0.2) (layer "F.Cu") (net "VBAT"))
 (segment (start 143.5 66) (end 143.75 66.25) (width 0.2) (layer "F.Cu") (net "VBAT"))
 (segment (start 133.47 59.3) (end 134.7 59.3) (width 0.2) (layer "F.Cu") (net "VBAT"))
 (segment (start 141.790256 66) (end 143.5 66) (width 0.2) (layer "F.Cu") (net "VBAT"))
 (segment (start 143.75 67.25) (end 143.5 67.5) (width 0.2) (layer "F.Cu") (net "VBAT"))
 (segment (start 147.55 67.5) (end 145 67.5) (width 0.2) (layer "F.Cu") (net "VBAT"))
 (segment (start 143.5 66) (end 145 67.5) (width 0.2) (layer "F.Cu") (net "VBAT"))
 (segment (start 140.465255 67.325001) (end 141.790256 66) (width 0.2) (layer "F.Cu") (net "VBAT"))
 (segment (start 129.5 49.46) (end 129.5 52) (width 0.2) (layer "F.Cu") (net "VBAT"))
 (segment (start 134.7 59.3) (end 135 59) (width 0.2) (layer "F.Cu") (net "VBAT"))
 (segment (start 139.421 67.325001) (end 140.465255 67.325001) (width 0.2) (layer "F.Cu") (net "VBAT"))
 (via (at 143.5 67.5) (size 0.6) (drill 0.3) (layers "F.Cu" "B.Cu") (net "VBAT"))
 (via (at 135 59) (size 0.6) (drill 0.3) (layers "F.Cu" "B.Cu") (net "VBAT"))
 (segment (start 143.434635 59.6507) (end 144.0493 60.265365) (width 0.2) (layer "B.Cu") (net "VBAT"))
 (segment (start 135 59) (end 135.6507 59.6507) (width 0.2) (layer "B.Cu") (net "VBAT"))
 (segment (start 135 54.96) (end 128.54 48.5) (width 0.2) (layer "B.Cu") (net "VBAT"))
 (segment (start 135.6507 59.6507) (end 143.434635 59.6507) (width 0.2) (layer "B.Cu") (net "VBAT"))
 (segment (start 135 59) (end 135 54.96) (width 0.2) (layer "B.Cu") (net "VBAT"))
 (segment (start 144.0493 60.265365) (end 144.0493 66.9507) (width 0.2) (layer "B.Cu") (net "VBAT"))
 (segment (start 144.0493 66.9507) (end 143.5 67.5) (width 0.2) (layer "B.Cu") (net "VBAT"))
 (segment (start 141.575001 67.974999) (end 142.05 67.5) (width 0.2) (layer "F.Cu") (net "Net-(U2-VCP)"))
 (segment (start 139.421 67.974999) (end 141.575001 67.974999) (width 0.2) (layer "F.Cu") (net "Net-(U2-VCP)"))
 (segment (start 139.5 57) (end 139.5 62.075) (width 0.2) (layer "F.Cu") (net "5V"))
 (segment (start 135 64.92764) (end 135.514047 65.441687) (width 0.2) (layer "F.Cu") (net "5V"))
 (segment (start 155.925 67.5) (end 155.925 63.615) (width 0.2) (layer "F.Cu") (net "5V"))
 (segment (start 139.5 62.075) (end 139.925 62.5) (width 0.2) (layer "F.Cu") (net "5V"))
 (segment (start 135 64.725001) (end 135 64.92764) (width 0.2) (layer "F.Cu") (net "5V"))
 (segment (start 158.5 51) (end 159.65 52.15) (width 0.2) (layer "F.Cu") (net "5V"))
 (segment (start 129.5 57) (end 133.47 57) (width 0.2) (layer "F.Cu") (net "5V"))
 (segment (start 138.54 50.54) (end 140.46 50.54) (width 0.2) (layer "F.Cu") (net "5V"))
 (segment (start 159.65 59.89) (end 158.5 61.04) (width 0.2) (layer "F.Cu") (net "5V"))
 (segment (start 128 69.1875) (end 128.2625 68.925) (width 0.2) (layer "F.Cu") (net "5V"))
 (segment (start 140.46 50.54) (end 143 48) (width 0.2) (layer "F.Cu") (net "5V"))
 (segment (start 139.5 51.5) (end 139.5 57) (width 0.2) (layer "F.Cu") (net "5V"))
 (segment (start 155.925 63.615) (end 158.5 61.04) (width 0.2) (layer "F.Cu") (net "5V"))
 (segment (start 137.699999 64.725001) (end 135 64.725001) (width 0.2) (layer "F.Cu") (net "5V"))
 (segment (start 139.925 62.5) (end 137.699999 64.725001) (width 0.2) (layer "F.Cu") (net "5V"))
 (segment (start 133.47 57) (end 139.5 57) (width 0.2) (layer "F.Cu") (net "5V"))
 (segment (start 159.65 52.15) (end 159.65 59.89) (width 0.2) (layer "F.Cu") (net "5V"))
 (segment (start 138.54 50.54) (end 139.5 51.5) (width 0.2) (layer "F.Cu") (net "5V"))
 (segment (start 128.2625 68.925) (end 130 68.925) (width 0.2) (layer "F.Cu") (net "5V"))
 (segment (start 135 64.725001) (end 133.579 64.725001) (width 0.2) (layer "F.Cu") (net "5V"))
 (via (at 135.514047 65.441687) (size 0.6) (drill 0.3) (layers "F.Cu" "B.Cu") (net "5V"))
 (via (at 128 69.1875) (size 0.6) (drill 0.3) (layers "F.Cu" "B.Cu") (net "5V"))
 (segment (start 135.514047 65.441687) (end 134.97236 64.9) (width 0.2) (layer "B.Cu") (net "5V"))
 (segment (start 127.751471 64.9) (end 127.4 65.251471) (width 0.2) (layer "B.Cu") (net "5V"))
 (segment (start 144.0493 49.0493) (end 156.5493 49.0493) (width 0.2) (layer "B.Cu") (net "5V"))
 (segment (start 127.4 68.5875) (end 128 69.1875) (width 0.2) (layer "B.Cu") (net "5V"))
 (segment (start 143 48) (end 144.0493 49.0493) (width 0.2) (layer "B.Cu") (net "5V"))
 (segment (start 127.4 65.251471) (end 127.4 68.5875) (width 0.2) (layer "B.Cu") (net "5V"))
 (segment (start 156.5493 49.0493) (end 158.5 51) (width 0.2) (layer "B.Cu") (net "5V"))
 (segment (start 134.97236 64.9) (end 127.751471 64.9) (width 0.2) (layer "B.Cu") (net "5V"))
 (segment (start 150.62 53.08) (end 158.04 53.08) (width 0.2) (layer "B.Cu") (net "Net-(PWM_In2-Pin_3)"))
 (segment (start 158.04 53.08) (end 158.5 53.54) (width 0.2) (layer "B.Cu") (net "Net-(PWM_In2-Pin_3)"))
 (segment (start 146.9575 57.0375) (end 143 53.08) (width 0.2) (layer "F.Cu") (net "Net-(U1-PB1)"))
 (segment (start 154 57.0375) (end 146.9575 57.0375) (width 0.2) (layer "F.Cu") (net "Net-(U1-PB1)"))
 (segment (start 154 62) (end 154 59.9625) (width 0.2) (layer "F.Cu") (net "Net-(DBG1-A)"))
 (segment (start 133.5 62.5) (end 137 62.5) (width 0.2) (layer "F.Cu") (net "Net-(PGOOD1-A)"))
 (segment (start 127.5 66) (end 126 66) (width 0.2) (layer "F.Cu") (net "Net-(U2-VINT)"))
 (segment (start 138.025001 66.025001) (end 137.5 65.5) (width 0.2) (layer "F.Cu") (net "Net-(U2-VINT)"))
 (segment (start 128 65.5) (end 127.5 66) (width 0.2) (layer "F.Cu") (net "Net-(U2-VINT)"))
 (segment (start 139.421 66.025001) (end 138.025001 66.025001) (width 0.2) (layer "F.Cu") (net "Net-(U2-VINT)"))
 (via (at 128 65.5) (size 0.6) (drill 0.3) (layers "F.Cu" "B.Cu") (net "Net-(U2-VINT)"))
 (via (at 137.5 65.5) (size 0.6) (drill 0.3) (layers "F.Cu" "B.Cu") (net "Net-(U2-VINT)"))
 (segment (start 135.748529 67.6) (end 130.1 67.6) (width 0.2) (layer "B.Cu") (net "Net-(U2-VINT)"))
 (segment (start 137.5 65.848529) (end 135.748529 67.6) (width 0.2) (layer "B.Cu") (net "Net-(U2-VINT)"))
 (segment (start 137.5 65.5) (end 137.5 65.848529) (width 0.2) (layer "B.Cu") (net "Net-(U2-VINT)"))
 (segment (start 130.1 67.6) (end 128 65.5) (width 0.2) (layer "B.Cu") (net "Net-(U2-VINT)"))
 (segment (start 153 67.5) (end 147.4507 61.9507) (width 0.2) (layer "F.Cu") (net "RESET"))
 (segment (start 147.4507 61.9507) (end 147.4507 60.0707) (width 0.2) (layer "F.Cu") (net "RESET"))
 (segment (start 147.4507 60.0707) (end 143 55.62) (width 0.2) (layer "F.Cu") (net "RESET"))
 (segment (start 141.993654 55.62) (end 143 55.62) (width 0.2) (layer "B.Cu") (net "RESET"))
 (segment (start 137.39 51.016346) (end 141.993654 55.62) (width 0.2) (layer "B.Cu") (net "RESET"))
 (segment (start 137.39 50.063654) (end 137.39 51.016346) (width 0.2) (layer "B.Cu") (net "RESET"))
 (segment (start 136.476346 49.15) (end 137.39 50.063654) (width 0.2) (layer "B.Cu") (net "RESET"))
 (segment (start 133.46 48) (end 134.61 49.15) (width 0.2) (layer "B.Cu") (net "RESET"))
 (segment (start 134.61 49.15) (end 136.476346 49.15) (width 0.2) (layer "B.Cu") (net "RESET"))
 (segment (start 130 64) (end 131.5 64) (width 0.2) (layer "F.Cu") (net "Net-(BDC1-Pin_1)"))
 (segment (start 132.874999 65.374999) (end 133.579 65.374999) (width 0.2) (layer "F.Cu") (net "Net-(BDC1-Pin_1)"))
 (segment (start 131.5 64) (end 132.874999 65.374999) (width 0.2) (layer "F.Cu") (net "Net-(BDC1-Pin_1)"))
 (segment (start 126 60) (end 130 64) (width 0.2) (layer "F.Cu") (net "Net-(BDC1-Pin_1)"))
 (segment (start 132.6424 66.674999) (end 133.579 66.674999) (width 0.2) (layer "F.Cu") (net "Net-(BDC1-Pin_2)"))
 (segment (start 131.104901 65.1375) (end 132.6424 66.674999) (width 0.2) (layer "F.Cu") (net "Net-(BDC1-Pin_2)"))
 (segment (start 126 62.54) (end 128.5975 65.1375) (width 0.2) (layer "F.Cu") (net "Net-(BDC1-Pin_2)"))
 (segment (start 128.5975 65.1375) (end 131.104901 65.1375) (width 0.2) (layer "F.Cu") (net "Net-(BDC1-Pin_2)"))
 (segment (start 133.579 67.324998) (end 135.175002 67.324998) (width 0.2) (layer "F.Cu") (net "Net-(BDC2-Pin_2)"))
 (segment (start 135.175002 67.324998) (end 135.5 67) (width 0.2) (layer "F.Cu") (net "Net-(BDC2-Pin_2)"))
 (via (at 135.5 67) (size 0.6) (drill 0.3) (layers "F.Cu" "B.Cu") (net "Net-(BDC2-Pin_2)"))
 (segment (start 135.5 67) (end 136.114047 66.385953) (width 0.2) (layer "B.Cu") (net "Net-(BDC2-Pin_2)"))
 (segment (start 136.114047 66.385953) (end 136.114047 65.193158) (width 0.2) (layer "B.Cu") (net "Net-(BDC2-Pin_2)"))
 (segment (start 136.114047 65.193158) (end 126.460889 55.54) (width 0.2) (layer "B.Cu") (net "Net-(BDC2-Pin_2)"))
 (segment (start 126.460889 55.54) (end 126 55.54) (width 0.2) (layer "B.Cu") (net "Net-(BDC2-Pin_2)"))
 (segment (start 133.579 68.624998) (end 135.450001 68.624998) (width 0.2) (layer "F.Cu") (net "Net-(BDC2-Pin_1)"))
 (segment (start 135.450001 68.624998) (end 135.5 68.574999) (width 0.2) (layer "F.Cu") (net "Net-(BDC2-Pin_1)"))
 (via (at 135.5 68.574999) (size 0.6) (drill 0.3) (layers "F.Cu" "B.Cu") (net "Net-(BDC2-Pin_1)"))
 (segment (start 135.5 68.574999) (end 138.1 65.974999) (width 0.2) (layer "B.Cu") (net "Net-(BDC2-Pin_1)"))
 (segment (start 138.1 65.974999) (end 138.1 65.1) (width 0.2) (layer "B.Cu") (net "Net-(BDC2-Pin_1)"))
 (segment (start 138.1 65.1) (end 126 53) (width 0.2) (layer "B.Cu") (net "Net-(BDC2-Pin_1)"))
 (segment (start 132.712499 69.274999) (end 133.579 69.274999) (width 0.2) (layer "F.Cu") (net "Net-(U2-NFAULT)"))
 (segment (start 130 66) (end 130 66.5625) (width 0.2) (layer "F.Cu") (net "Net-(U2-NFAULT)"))
 (segment (start 130 66.5625) (end 132.712499 69.274999) (width 0.2) (layer "F.Cu") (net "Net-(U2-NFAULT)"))
 (segment (start 137.5 69) (end 137.774999 69.274999) (width 0.2) (layer "F.Cu") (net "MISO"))
 (segment (start 137.774999 69.274999) (end 139.421 69.274999) (width 0.2) (layer "F.Cu") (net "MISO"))
 (via (at 137.5 69) (size 0.6) (drill 0.3) (layers "F.Cu" "B.Cu") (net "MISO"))
 (segment (start 148.1 60.72) (end 148.1 56.696065) (width 0.2) (layer "B.Cu") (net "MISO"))
 (segment (start 150.62 63.24) (end 148.1 60.72) (width 0.2) (layer "B.Cu") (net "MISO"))
 (segment (start 150.62 63.24) (end 144.86 69) (width 0.2) (layer "B.Cu") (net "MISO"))
 (segment (start 144.86 69) (end 137.5 69) (width 0.2) (layer "B.Cu") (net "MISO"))
 (segment (start 148.1 56.696065) (end 143.403935 52) (width 0.2) (layer "B.Cu") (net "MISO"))
 (segment (start 143.403935 52) (end 142.54 52) (width 0.2) (layer "B.Cu") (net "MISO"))
 (segment (start 142.54 52) (end 138.54 48) (width 0.2) (layer "B.Cu") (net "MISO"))
 (segment (start 138.180128 67.9) (end 138.180128 68.248527) (width 0.2) (layer "F.Cu") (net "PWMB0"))
 (segment (start 138.556602 68.625001) (end 139.421 68.625001) (width 0.2) (layer "F.Cu") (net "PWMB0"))
 (segment (start 138.180128 68.248527) (end 138.556602 68.625001) (width 0.2) (layer "F.Cu") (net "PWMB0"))
 (via (at 138.180128 67.9) (size 0.6) (drill 0.3) (layers "F.Cu" "B.Cu") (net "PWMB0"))
 (segment (start 141.9507 64.129428) (end 138.180128 67.9) (width 0.2) (layer "B.Cu") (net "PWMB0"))
 (segment (start 143 60.7) (end 141.9507 61.7493) (width 0.2) (layer "B.Cu") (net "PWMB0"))
 (segment (start 141.9507 61.7493) (end 141.9507 64.129428) (width 0.2) (layer "B.Cu") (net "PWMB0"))
 (segment (start 145 62.5) (end 144.26 63.24) (width 0.2) (layer "F.Cu") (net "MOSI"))
 (segment (start 143 63.24) (end 140.864998 65.375002) (width 0.2) (layer "F.Cu") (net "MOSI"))
 (segment (start 140.864998 65.375002) (end 139.421 65.375002) (width 0.2) (layer "F.Cu") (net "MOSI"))
 (segment (start 144.26 63.24) (end 143 63.24) (width 0.2) (layer "F.Cu") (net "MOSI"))
 (via (at 145 62.5) (size 0.6) (drill 0.3) (layers "F.Cu" "B.Cu") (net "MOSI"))
 (segment (start 143.600321 59.2507) (end 145 60.650379) (width 0.2) (layer "B.Cu") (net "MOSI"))
 (segment (start 136 50.54) (end 136 53) (width 0.2) (layer "B.Cu") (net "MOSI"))
 (segment (start 142.2507 59.2507) (end 143.600321 59.2507) (width 0.2) (layer "B.Cu") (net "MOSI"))
 (segment (start 145 60.650379) (end 145 62.5) (width 0.2) (layer "B.Cu") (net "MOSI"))
 (segment (start 136 53) (end 142.2507 59.2507) (width 0.2) (layer "B.Cu") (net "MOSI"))
 (segment (start 141.5 59.66) (end 141.5 63.204801) (width 0.2) (layer "F.Cu") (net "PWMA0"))
 (segment (start 141.5 63.204801) (end 139.9798 64.725001) (width 0.2) (layer "F.Cu") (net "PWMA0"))
 (segment (start 143 58.16) (end 141.5 59.66) (width 0.2) (layer "F.Cu") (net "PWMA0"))
 (segment (start 139.9798 64.725001) (end 139.421 64.725001) (width 0.2) (layer "F.Cu") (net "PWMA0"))
 (segment (start 150.62 60.7) (end 148.42 58.5) (width 0.2) (layer "F.Cu") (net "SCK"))
 (segment (start 148.42 58.5) (end 147.5 58.5) (width 0.2) (layer "F.Cu") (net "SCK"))
 (via (at 147.5 58.5) (size 0.6) (drill 0.3) (layers "F.Cu" "B.Cu") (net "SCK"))
 (segment (start 143.1293 54.1293) (end 142.565365 54.1293) (width 0.2) (layer "B.Cu") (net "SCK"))
 (segment (start 147.5 58.5) (end 143.1293 54.1293) (width 0.2) (layer "B.Cu") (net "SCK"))
 (segment (start 138.776346 49.15) (end 137.15 49.15) (width 0.2) (layer "B.Cu") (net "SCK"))
 (segment (start 139.69 51.253935) (end 139.69 50.063654) (width 0.2) (layer "B.Cu") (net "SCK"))
 (segment (start 137.15 49.15) (end 136 48) (width 0.2) (layer "B.Cu") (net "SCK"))
 (segment (start 139.69 50.063654) (end 138.776346 49.15) (width 0.2) (layer "B.Cu") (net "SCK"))
 (segment (start 142.565365 54.1293) (end 139.69 51.253935) (width 0.2) (layer "B.Cu") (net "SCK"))
 (segment (start 154 52) (end 154 50) (width 0.2) (layer "F.Cu") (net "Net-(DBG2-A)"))
 (segment (start 150.6107 57.1107) (end 152.0307 57.1107) (width 0.2) (layer "B.Cu") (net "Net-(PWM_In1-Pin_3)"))
 (segment (start 150.611471 50.54) (end 147.9 53.251471) (width 0.2) (layer "B.Cu") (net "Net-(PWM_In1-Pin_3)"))
 (segment (start 147.9 54.4) (end 150.6107 57.1107) (width 0.2) (layer "B.Cu") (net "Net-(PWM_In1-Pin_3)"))
 (segment (start 147.9 53.251471) (end 147.9 54.4) (width 0.2) (layer "B.Cu") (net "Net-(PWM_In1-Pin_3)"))
 (segment (start 152.0307 57.1107) (end 158.5 63.58) (width 0.2) (layer "B.Cu") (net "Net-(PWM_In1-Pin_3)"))
 (segment (start 150.62 50.54) (end 150.611471 50.54) (width 0.2) (layer "B.Cu") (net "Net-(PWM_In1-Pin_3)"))
 (segment (start 144.0493 49.4907) (end 143 50.54) (width 0.2) (layer "F.Cu") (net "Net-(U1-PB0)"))
 (segment (start 151.5843 49.4907) (end 144.0493 49.4907) (width 0.2) (layer "F.Cu") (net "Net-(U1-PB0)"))
 (segment (start 154 47.075) (end 151.5843 49.4907) (width 0.2) (layer "F.Cu") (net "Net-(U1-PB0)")))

